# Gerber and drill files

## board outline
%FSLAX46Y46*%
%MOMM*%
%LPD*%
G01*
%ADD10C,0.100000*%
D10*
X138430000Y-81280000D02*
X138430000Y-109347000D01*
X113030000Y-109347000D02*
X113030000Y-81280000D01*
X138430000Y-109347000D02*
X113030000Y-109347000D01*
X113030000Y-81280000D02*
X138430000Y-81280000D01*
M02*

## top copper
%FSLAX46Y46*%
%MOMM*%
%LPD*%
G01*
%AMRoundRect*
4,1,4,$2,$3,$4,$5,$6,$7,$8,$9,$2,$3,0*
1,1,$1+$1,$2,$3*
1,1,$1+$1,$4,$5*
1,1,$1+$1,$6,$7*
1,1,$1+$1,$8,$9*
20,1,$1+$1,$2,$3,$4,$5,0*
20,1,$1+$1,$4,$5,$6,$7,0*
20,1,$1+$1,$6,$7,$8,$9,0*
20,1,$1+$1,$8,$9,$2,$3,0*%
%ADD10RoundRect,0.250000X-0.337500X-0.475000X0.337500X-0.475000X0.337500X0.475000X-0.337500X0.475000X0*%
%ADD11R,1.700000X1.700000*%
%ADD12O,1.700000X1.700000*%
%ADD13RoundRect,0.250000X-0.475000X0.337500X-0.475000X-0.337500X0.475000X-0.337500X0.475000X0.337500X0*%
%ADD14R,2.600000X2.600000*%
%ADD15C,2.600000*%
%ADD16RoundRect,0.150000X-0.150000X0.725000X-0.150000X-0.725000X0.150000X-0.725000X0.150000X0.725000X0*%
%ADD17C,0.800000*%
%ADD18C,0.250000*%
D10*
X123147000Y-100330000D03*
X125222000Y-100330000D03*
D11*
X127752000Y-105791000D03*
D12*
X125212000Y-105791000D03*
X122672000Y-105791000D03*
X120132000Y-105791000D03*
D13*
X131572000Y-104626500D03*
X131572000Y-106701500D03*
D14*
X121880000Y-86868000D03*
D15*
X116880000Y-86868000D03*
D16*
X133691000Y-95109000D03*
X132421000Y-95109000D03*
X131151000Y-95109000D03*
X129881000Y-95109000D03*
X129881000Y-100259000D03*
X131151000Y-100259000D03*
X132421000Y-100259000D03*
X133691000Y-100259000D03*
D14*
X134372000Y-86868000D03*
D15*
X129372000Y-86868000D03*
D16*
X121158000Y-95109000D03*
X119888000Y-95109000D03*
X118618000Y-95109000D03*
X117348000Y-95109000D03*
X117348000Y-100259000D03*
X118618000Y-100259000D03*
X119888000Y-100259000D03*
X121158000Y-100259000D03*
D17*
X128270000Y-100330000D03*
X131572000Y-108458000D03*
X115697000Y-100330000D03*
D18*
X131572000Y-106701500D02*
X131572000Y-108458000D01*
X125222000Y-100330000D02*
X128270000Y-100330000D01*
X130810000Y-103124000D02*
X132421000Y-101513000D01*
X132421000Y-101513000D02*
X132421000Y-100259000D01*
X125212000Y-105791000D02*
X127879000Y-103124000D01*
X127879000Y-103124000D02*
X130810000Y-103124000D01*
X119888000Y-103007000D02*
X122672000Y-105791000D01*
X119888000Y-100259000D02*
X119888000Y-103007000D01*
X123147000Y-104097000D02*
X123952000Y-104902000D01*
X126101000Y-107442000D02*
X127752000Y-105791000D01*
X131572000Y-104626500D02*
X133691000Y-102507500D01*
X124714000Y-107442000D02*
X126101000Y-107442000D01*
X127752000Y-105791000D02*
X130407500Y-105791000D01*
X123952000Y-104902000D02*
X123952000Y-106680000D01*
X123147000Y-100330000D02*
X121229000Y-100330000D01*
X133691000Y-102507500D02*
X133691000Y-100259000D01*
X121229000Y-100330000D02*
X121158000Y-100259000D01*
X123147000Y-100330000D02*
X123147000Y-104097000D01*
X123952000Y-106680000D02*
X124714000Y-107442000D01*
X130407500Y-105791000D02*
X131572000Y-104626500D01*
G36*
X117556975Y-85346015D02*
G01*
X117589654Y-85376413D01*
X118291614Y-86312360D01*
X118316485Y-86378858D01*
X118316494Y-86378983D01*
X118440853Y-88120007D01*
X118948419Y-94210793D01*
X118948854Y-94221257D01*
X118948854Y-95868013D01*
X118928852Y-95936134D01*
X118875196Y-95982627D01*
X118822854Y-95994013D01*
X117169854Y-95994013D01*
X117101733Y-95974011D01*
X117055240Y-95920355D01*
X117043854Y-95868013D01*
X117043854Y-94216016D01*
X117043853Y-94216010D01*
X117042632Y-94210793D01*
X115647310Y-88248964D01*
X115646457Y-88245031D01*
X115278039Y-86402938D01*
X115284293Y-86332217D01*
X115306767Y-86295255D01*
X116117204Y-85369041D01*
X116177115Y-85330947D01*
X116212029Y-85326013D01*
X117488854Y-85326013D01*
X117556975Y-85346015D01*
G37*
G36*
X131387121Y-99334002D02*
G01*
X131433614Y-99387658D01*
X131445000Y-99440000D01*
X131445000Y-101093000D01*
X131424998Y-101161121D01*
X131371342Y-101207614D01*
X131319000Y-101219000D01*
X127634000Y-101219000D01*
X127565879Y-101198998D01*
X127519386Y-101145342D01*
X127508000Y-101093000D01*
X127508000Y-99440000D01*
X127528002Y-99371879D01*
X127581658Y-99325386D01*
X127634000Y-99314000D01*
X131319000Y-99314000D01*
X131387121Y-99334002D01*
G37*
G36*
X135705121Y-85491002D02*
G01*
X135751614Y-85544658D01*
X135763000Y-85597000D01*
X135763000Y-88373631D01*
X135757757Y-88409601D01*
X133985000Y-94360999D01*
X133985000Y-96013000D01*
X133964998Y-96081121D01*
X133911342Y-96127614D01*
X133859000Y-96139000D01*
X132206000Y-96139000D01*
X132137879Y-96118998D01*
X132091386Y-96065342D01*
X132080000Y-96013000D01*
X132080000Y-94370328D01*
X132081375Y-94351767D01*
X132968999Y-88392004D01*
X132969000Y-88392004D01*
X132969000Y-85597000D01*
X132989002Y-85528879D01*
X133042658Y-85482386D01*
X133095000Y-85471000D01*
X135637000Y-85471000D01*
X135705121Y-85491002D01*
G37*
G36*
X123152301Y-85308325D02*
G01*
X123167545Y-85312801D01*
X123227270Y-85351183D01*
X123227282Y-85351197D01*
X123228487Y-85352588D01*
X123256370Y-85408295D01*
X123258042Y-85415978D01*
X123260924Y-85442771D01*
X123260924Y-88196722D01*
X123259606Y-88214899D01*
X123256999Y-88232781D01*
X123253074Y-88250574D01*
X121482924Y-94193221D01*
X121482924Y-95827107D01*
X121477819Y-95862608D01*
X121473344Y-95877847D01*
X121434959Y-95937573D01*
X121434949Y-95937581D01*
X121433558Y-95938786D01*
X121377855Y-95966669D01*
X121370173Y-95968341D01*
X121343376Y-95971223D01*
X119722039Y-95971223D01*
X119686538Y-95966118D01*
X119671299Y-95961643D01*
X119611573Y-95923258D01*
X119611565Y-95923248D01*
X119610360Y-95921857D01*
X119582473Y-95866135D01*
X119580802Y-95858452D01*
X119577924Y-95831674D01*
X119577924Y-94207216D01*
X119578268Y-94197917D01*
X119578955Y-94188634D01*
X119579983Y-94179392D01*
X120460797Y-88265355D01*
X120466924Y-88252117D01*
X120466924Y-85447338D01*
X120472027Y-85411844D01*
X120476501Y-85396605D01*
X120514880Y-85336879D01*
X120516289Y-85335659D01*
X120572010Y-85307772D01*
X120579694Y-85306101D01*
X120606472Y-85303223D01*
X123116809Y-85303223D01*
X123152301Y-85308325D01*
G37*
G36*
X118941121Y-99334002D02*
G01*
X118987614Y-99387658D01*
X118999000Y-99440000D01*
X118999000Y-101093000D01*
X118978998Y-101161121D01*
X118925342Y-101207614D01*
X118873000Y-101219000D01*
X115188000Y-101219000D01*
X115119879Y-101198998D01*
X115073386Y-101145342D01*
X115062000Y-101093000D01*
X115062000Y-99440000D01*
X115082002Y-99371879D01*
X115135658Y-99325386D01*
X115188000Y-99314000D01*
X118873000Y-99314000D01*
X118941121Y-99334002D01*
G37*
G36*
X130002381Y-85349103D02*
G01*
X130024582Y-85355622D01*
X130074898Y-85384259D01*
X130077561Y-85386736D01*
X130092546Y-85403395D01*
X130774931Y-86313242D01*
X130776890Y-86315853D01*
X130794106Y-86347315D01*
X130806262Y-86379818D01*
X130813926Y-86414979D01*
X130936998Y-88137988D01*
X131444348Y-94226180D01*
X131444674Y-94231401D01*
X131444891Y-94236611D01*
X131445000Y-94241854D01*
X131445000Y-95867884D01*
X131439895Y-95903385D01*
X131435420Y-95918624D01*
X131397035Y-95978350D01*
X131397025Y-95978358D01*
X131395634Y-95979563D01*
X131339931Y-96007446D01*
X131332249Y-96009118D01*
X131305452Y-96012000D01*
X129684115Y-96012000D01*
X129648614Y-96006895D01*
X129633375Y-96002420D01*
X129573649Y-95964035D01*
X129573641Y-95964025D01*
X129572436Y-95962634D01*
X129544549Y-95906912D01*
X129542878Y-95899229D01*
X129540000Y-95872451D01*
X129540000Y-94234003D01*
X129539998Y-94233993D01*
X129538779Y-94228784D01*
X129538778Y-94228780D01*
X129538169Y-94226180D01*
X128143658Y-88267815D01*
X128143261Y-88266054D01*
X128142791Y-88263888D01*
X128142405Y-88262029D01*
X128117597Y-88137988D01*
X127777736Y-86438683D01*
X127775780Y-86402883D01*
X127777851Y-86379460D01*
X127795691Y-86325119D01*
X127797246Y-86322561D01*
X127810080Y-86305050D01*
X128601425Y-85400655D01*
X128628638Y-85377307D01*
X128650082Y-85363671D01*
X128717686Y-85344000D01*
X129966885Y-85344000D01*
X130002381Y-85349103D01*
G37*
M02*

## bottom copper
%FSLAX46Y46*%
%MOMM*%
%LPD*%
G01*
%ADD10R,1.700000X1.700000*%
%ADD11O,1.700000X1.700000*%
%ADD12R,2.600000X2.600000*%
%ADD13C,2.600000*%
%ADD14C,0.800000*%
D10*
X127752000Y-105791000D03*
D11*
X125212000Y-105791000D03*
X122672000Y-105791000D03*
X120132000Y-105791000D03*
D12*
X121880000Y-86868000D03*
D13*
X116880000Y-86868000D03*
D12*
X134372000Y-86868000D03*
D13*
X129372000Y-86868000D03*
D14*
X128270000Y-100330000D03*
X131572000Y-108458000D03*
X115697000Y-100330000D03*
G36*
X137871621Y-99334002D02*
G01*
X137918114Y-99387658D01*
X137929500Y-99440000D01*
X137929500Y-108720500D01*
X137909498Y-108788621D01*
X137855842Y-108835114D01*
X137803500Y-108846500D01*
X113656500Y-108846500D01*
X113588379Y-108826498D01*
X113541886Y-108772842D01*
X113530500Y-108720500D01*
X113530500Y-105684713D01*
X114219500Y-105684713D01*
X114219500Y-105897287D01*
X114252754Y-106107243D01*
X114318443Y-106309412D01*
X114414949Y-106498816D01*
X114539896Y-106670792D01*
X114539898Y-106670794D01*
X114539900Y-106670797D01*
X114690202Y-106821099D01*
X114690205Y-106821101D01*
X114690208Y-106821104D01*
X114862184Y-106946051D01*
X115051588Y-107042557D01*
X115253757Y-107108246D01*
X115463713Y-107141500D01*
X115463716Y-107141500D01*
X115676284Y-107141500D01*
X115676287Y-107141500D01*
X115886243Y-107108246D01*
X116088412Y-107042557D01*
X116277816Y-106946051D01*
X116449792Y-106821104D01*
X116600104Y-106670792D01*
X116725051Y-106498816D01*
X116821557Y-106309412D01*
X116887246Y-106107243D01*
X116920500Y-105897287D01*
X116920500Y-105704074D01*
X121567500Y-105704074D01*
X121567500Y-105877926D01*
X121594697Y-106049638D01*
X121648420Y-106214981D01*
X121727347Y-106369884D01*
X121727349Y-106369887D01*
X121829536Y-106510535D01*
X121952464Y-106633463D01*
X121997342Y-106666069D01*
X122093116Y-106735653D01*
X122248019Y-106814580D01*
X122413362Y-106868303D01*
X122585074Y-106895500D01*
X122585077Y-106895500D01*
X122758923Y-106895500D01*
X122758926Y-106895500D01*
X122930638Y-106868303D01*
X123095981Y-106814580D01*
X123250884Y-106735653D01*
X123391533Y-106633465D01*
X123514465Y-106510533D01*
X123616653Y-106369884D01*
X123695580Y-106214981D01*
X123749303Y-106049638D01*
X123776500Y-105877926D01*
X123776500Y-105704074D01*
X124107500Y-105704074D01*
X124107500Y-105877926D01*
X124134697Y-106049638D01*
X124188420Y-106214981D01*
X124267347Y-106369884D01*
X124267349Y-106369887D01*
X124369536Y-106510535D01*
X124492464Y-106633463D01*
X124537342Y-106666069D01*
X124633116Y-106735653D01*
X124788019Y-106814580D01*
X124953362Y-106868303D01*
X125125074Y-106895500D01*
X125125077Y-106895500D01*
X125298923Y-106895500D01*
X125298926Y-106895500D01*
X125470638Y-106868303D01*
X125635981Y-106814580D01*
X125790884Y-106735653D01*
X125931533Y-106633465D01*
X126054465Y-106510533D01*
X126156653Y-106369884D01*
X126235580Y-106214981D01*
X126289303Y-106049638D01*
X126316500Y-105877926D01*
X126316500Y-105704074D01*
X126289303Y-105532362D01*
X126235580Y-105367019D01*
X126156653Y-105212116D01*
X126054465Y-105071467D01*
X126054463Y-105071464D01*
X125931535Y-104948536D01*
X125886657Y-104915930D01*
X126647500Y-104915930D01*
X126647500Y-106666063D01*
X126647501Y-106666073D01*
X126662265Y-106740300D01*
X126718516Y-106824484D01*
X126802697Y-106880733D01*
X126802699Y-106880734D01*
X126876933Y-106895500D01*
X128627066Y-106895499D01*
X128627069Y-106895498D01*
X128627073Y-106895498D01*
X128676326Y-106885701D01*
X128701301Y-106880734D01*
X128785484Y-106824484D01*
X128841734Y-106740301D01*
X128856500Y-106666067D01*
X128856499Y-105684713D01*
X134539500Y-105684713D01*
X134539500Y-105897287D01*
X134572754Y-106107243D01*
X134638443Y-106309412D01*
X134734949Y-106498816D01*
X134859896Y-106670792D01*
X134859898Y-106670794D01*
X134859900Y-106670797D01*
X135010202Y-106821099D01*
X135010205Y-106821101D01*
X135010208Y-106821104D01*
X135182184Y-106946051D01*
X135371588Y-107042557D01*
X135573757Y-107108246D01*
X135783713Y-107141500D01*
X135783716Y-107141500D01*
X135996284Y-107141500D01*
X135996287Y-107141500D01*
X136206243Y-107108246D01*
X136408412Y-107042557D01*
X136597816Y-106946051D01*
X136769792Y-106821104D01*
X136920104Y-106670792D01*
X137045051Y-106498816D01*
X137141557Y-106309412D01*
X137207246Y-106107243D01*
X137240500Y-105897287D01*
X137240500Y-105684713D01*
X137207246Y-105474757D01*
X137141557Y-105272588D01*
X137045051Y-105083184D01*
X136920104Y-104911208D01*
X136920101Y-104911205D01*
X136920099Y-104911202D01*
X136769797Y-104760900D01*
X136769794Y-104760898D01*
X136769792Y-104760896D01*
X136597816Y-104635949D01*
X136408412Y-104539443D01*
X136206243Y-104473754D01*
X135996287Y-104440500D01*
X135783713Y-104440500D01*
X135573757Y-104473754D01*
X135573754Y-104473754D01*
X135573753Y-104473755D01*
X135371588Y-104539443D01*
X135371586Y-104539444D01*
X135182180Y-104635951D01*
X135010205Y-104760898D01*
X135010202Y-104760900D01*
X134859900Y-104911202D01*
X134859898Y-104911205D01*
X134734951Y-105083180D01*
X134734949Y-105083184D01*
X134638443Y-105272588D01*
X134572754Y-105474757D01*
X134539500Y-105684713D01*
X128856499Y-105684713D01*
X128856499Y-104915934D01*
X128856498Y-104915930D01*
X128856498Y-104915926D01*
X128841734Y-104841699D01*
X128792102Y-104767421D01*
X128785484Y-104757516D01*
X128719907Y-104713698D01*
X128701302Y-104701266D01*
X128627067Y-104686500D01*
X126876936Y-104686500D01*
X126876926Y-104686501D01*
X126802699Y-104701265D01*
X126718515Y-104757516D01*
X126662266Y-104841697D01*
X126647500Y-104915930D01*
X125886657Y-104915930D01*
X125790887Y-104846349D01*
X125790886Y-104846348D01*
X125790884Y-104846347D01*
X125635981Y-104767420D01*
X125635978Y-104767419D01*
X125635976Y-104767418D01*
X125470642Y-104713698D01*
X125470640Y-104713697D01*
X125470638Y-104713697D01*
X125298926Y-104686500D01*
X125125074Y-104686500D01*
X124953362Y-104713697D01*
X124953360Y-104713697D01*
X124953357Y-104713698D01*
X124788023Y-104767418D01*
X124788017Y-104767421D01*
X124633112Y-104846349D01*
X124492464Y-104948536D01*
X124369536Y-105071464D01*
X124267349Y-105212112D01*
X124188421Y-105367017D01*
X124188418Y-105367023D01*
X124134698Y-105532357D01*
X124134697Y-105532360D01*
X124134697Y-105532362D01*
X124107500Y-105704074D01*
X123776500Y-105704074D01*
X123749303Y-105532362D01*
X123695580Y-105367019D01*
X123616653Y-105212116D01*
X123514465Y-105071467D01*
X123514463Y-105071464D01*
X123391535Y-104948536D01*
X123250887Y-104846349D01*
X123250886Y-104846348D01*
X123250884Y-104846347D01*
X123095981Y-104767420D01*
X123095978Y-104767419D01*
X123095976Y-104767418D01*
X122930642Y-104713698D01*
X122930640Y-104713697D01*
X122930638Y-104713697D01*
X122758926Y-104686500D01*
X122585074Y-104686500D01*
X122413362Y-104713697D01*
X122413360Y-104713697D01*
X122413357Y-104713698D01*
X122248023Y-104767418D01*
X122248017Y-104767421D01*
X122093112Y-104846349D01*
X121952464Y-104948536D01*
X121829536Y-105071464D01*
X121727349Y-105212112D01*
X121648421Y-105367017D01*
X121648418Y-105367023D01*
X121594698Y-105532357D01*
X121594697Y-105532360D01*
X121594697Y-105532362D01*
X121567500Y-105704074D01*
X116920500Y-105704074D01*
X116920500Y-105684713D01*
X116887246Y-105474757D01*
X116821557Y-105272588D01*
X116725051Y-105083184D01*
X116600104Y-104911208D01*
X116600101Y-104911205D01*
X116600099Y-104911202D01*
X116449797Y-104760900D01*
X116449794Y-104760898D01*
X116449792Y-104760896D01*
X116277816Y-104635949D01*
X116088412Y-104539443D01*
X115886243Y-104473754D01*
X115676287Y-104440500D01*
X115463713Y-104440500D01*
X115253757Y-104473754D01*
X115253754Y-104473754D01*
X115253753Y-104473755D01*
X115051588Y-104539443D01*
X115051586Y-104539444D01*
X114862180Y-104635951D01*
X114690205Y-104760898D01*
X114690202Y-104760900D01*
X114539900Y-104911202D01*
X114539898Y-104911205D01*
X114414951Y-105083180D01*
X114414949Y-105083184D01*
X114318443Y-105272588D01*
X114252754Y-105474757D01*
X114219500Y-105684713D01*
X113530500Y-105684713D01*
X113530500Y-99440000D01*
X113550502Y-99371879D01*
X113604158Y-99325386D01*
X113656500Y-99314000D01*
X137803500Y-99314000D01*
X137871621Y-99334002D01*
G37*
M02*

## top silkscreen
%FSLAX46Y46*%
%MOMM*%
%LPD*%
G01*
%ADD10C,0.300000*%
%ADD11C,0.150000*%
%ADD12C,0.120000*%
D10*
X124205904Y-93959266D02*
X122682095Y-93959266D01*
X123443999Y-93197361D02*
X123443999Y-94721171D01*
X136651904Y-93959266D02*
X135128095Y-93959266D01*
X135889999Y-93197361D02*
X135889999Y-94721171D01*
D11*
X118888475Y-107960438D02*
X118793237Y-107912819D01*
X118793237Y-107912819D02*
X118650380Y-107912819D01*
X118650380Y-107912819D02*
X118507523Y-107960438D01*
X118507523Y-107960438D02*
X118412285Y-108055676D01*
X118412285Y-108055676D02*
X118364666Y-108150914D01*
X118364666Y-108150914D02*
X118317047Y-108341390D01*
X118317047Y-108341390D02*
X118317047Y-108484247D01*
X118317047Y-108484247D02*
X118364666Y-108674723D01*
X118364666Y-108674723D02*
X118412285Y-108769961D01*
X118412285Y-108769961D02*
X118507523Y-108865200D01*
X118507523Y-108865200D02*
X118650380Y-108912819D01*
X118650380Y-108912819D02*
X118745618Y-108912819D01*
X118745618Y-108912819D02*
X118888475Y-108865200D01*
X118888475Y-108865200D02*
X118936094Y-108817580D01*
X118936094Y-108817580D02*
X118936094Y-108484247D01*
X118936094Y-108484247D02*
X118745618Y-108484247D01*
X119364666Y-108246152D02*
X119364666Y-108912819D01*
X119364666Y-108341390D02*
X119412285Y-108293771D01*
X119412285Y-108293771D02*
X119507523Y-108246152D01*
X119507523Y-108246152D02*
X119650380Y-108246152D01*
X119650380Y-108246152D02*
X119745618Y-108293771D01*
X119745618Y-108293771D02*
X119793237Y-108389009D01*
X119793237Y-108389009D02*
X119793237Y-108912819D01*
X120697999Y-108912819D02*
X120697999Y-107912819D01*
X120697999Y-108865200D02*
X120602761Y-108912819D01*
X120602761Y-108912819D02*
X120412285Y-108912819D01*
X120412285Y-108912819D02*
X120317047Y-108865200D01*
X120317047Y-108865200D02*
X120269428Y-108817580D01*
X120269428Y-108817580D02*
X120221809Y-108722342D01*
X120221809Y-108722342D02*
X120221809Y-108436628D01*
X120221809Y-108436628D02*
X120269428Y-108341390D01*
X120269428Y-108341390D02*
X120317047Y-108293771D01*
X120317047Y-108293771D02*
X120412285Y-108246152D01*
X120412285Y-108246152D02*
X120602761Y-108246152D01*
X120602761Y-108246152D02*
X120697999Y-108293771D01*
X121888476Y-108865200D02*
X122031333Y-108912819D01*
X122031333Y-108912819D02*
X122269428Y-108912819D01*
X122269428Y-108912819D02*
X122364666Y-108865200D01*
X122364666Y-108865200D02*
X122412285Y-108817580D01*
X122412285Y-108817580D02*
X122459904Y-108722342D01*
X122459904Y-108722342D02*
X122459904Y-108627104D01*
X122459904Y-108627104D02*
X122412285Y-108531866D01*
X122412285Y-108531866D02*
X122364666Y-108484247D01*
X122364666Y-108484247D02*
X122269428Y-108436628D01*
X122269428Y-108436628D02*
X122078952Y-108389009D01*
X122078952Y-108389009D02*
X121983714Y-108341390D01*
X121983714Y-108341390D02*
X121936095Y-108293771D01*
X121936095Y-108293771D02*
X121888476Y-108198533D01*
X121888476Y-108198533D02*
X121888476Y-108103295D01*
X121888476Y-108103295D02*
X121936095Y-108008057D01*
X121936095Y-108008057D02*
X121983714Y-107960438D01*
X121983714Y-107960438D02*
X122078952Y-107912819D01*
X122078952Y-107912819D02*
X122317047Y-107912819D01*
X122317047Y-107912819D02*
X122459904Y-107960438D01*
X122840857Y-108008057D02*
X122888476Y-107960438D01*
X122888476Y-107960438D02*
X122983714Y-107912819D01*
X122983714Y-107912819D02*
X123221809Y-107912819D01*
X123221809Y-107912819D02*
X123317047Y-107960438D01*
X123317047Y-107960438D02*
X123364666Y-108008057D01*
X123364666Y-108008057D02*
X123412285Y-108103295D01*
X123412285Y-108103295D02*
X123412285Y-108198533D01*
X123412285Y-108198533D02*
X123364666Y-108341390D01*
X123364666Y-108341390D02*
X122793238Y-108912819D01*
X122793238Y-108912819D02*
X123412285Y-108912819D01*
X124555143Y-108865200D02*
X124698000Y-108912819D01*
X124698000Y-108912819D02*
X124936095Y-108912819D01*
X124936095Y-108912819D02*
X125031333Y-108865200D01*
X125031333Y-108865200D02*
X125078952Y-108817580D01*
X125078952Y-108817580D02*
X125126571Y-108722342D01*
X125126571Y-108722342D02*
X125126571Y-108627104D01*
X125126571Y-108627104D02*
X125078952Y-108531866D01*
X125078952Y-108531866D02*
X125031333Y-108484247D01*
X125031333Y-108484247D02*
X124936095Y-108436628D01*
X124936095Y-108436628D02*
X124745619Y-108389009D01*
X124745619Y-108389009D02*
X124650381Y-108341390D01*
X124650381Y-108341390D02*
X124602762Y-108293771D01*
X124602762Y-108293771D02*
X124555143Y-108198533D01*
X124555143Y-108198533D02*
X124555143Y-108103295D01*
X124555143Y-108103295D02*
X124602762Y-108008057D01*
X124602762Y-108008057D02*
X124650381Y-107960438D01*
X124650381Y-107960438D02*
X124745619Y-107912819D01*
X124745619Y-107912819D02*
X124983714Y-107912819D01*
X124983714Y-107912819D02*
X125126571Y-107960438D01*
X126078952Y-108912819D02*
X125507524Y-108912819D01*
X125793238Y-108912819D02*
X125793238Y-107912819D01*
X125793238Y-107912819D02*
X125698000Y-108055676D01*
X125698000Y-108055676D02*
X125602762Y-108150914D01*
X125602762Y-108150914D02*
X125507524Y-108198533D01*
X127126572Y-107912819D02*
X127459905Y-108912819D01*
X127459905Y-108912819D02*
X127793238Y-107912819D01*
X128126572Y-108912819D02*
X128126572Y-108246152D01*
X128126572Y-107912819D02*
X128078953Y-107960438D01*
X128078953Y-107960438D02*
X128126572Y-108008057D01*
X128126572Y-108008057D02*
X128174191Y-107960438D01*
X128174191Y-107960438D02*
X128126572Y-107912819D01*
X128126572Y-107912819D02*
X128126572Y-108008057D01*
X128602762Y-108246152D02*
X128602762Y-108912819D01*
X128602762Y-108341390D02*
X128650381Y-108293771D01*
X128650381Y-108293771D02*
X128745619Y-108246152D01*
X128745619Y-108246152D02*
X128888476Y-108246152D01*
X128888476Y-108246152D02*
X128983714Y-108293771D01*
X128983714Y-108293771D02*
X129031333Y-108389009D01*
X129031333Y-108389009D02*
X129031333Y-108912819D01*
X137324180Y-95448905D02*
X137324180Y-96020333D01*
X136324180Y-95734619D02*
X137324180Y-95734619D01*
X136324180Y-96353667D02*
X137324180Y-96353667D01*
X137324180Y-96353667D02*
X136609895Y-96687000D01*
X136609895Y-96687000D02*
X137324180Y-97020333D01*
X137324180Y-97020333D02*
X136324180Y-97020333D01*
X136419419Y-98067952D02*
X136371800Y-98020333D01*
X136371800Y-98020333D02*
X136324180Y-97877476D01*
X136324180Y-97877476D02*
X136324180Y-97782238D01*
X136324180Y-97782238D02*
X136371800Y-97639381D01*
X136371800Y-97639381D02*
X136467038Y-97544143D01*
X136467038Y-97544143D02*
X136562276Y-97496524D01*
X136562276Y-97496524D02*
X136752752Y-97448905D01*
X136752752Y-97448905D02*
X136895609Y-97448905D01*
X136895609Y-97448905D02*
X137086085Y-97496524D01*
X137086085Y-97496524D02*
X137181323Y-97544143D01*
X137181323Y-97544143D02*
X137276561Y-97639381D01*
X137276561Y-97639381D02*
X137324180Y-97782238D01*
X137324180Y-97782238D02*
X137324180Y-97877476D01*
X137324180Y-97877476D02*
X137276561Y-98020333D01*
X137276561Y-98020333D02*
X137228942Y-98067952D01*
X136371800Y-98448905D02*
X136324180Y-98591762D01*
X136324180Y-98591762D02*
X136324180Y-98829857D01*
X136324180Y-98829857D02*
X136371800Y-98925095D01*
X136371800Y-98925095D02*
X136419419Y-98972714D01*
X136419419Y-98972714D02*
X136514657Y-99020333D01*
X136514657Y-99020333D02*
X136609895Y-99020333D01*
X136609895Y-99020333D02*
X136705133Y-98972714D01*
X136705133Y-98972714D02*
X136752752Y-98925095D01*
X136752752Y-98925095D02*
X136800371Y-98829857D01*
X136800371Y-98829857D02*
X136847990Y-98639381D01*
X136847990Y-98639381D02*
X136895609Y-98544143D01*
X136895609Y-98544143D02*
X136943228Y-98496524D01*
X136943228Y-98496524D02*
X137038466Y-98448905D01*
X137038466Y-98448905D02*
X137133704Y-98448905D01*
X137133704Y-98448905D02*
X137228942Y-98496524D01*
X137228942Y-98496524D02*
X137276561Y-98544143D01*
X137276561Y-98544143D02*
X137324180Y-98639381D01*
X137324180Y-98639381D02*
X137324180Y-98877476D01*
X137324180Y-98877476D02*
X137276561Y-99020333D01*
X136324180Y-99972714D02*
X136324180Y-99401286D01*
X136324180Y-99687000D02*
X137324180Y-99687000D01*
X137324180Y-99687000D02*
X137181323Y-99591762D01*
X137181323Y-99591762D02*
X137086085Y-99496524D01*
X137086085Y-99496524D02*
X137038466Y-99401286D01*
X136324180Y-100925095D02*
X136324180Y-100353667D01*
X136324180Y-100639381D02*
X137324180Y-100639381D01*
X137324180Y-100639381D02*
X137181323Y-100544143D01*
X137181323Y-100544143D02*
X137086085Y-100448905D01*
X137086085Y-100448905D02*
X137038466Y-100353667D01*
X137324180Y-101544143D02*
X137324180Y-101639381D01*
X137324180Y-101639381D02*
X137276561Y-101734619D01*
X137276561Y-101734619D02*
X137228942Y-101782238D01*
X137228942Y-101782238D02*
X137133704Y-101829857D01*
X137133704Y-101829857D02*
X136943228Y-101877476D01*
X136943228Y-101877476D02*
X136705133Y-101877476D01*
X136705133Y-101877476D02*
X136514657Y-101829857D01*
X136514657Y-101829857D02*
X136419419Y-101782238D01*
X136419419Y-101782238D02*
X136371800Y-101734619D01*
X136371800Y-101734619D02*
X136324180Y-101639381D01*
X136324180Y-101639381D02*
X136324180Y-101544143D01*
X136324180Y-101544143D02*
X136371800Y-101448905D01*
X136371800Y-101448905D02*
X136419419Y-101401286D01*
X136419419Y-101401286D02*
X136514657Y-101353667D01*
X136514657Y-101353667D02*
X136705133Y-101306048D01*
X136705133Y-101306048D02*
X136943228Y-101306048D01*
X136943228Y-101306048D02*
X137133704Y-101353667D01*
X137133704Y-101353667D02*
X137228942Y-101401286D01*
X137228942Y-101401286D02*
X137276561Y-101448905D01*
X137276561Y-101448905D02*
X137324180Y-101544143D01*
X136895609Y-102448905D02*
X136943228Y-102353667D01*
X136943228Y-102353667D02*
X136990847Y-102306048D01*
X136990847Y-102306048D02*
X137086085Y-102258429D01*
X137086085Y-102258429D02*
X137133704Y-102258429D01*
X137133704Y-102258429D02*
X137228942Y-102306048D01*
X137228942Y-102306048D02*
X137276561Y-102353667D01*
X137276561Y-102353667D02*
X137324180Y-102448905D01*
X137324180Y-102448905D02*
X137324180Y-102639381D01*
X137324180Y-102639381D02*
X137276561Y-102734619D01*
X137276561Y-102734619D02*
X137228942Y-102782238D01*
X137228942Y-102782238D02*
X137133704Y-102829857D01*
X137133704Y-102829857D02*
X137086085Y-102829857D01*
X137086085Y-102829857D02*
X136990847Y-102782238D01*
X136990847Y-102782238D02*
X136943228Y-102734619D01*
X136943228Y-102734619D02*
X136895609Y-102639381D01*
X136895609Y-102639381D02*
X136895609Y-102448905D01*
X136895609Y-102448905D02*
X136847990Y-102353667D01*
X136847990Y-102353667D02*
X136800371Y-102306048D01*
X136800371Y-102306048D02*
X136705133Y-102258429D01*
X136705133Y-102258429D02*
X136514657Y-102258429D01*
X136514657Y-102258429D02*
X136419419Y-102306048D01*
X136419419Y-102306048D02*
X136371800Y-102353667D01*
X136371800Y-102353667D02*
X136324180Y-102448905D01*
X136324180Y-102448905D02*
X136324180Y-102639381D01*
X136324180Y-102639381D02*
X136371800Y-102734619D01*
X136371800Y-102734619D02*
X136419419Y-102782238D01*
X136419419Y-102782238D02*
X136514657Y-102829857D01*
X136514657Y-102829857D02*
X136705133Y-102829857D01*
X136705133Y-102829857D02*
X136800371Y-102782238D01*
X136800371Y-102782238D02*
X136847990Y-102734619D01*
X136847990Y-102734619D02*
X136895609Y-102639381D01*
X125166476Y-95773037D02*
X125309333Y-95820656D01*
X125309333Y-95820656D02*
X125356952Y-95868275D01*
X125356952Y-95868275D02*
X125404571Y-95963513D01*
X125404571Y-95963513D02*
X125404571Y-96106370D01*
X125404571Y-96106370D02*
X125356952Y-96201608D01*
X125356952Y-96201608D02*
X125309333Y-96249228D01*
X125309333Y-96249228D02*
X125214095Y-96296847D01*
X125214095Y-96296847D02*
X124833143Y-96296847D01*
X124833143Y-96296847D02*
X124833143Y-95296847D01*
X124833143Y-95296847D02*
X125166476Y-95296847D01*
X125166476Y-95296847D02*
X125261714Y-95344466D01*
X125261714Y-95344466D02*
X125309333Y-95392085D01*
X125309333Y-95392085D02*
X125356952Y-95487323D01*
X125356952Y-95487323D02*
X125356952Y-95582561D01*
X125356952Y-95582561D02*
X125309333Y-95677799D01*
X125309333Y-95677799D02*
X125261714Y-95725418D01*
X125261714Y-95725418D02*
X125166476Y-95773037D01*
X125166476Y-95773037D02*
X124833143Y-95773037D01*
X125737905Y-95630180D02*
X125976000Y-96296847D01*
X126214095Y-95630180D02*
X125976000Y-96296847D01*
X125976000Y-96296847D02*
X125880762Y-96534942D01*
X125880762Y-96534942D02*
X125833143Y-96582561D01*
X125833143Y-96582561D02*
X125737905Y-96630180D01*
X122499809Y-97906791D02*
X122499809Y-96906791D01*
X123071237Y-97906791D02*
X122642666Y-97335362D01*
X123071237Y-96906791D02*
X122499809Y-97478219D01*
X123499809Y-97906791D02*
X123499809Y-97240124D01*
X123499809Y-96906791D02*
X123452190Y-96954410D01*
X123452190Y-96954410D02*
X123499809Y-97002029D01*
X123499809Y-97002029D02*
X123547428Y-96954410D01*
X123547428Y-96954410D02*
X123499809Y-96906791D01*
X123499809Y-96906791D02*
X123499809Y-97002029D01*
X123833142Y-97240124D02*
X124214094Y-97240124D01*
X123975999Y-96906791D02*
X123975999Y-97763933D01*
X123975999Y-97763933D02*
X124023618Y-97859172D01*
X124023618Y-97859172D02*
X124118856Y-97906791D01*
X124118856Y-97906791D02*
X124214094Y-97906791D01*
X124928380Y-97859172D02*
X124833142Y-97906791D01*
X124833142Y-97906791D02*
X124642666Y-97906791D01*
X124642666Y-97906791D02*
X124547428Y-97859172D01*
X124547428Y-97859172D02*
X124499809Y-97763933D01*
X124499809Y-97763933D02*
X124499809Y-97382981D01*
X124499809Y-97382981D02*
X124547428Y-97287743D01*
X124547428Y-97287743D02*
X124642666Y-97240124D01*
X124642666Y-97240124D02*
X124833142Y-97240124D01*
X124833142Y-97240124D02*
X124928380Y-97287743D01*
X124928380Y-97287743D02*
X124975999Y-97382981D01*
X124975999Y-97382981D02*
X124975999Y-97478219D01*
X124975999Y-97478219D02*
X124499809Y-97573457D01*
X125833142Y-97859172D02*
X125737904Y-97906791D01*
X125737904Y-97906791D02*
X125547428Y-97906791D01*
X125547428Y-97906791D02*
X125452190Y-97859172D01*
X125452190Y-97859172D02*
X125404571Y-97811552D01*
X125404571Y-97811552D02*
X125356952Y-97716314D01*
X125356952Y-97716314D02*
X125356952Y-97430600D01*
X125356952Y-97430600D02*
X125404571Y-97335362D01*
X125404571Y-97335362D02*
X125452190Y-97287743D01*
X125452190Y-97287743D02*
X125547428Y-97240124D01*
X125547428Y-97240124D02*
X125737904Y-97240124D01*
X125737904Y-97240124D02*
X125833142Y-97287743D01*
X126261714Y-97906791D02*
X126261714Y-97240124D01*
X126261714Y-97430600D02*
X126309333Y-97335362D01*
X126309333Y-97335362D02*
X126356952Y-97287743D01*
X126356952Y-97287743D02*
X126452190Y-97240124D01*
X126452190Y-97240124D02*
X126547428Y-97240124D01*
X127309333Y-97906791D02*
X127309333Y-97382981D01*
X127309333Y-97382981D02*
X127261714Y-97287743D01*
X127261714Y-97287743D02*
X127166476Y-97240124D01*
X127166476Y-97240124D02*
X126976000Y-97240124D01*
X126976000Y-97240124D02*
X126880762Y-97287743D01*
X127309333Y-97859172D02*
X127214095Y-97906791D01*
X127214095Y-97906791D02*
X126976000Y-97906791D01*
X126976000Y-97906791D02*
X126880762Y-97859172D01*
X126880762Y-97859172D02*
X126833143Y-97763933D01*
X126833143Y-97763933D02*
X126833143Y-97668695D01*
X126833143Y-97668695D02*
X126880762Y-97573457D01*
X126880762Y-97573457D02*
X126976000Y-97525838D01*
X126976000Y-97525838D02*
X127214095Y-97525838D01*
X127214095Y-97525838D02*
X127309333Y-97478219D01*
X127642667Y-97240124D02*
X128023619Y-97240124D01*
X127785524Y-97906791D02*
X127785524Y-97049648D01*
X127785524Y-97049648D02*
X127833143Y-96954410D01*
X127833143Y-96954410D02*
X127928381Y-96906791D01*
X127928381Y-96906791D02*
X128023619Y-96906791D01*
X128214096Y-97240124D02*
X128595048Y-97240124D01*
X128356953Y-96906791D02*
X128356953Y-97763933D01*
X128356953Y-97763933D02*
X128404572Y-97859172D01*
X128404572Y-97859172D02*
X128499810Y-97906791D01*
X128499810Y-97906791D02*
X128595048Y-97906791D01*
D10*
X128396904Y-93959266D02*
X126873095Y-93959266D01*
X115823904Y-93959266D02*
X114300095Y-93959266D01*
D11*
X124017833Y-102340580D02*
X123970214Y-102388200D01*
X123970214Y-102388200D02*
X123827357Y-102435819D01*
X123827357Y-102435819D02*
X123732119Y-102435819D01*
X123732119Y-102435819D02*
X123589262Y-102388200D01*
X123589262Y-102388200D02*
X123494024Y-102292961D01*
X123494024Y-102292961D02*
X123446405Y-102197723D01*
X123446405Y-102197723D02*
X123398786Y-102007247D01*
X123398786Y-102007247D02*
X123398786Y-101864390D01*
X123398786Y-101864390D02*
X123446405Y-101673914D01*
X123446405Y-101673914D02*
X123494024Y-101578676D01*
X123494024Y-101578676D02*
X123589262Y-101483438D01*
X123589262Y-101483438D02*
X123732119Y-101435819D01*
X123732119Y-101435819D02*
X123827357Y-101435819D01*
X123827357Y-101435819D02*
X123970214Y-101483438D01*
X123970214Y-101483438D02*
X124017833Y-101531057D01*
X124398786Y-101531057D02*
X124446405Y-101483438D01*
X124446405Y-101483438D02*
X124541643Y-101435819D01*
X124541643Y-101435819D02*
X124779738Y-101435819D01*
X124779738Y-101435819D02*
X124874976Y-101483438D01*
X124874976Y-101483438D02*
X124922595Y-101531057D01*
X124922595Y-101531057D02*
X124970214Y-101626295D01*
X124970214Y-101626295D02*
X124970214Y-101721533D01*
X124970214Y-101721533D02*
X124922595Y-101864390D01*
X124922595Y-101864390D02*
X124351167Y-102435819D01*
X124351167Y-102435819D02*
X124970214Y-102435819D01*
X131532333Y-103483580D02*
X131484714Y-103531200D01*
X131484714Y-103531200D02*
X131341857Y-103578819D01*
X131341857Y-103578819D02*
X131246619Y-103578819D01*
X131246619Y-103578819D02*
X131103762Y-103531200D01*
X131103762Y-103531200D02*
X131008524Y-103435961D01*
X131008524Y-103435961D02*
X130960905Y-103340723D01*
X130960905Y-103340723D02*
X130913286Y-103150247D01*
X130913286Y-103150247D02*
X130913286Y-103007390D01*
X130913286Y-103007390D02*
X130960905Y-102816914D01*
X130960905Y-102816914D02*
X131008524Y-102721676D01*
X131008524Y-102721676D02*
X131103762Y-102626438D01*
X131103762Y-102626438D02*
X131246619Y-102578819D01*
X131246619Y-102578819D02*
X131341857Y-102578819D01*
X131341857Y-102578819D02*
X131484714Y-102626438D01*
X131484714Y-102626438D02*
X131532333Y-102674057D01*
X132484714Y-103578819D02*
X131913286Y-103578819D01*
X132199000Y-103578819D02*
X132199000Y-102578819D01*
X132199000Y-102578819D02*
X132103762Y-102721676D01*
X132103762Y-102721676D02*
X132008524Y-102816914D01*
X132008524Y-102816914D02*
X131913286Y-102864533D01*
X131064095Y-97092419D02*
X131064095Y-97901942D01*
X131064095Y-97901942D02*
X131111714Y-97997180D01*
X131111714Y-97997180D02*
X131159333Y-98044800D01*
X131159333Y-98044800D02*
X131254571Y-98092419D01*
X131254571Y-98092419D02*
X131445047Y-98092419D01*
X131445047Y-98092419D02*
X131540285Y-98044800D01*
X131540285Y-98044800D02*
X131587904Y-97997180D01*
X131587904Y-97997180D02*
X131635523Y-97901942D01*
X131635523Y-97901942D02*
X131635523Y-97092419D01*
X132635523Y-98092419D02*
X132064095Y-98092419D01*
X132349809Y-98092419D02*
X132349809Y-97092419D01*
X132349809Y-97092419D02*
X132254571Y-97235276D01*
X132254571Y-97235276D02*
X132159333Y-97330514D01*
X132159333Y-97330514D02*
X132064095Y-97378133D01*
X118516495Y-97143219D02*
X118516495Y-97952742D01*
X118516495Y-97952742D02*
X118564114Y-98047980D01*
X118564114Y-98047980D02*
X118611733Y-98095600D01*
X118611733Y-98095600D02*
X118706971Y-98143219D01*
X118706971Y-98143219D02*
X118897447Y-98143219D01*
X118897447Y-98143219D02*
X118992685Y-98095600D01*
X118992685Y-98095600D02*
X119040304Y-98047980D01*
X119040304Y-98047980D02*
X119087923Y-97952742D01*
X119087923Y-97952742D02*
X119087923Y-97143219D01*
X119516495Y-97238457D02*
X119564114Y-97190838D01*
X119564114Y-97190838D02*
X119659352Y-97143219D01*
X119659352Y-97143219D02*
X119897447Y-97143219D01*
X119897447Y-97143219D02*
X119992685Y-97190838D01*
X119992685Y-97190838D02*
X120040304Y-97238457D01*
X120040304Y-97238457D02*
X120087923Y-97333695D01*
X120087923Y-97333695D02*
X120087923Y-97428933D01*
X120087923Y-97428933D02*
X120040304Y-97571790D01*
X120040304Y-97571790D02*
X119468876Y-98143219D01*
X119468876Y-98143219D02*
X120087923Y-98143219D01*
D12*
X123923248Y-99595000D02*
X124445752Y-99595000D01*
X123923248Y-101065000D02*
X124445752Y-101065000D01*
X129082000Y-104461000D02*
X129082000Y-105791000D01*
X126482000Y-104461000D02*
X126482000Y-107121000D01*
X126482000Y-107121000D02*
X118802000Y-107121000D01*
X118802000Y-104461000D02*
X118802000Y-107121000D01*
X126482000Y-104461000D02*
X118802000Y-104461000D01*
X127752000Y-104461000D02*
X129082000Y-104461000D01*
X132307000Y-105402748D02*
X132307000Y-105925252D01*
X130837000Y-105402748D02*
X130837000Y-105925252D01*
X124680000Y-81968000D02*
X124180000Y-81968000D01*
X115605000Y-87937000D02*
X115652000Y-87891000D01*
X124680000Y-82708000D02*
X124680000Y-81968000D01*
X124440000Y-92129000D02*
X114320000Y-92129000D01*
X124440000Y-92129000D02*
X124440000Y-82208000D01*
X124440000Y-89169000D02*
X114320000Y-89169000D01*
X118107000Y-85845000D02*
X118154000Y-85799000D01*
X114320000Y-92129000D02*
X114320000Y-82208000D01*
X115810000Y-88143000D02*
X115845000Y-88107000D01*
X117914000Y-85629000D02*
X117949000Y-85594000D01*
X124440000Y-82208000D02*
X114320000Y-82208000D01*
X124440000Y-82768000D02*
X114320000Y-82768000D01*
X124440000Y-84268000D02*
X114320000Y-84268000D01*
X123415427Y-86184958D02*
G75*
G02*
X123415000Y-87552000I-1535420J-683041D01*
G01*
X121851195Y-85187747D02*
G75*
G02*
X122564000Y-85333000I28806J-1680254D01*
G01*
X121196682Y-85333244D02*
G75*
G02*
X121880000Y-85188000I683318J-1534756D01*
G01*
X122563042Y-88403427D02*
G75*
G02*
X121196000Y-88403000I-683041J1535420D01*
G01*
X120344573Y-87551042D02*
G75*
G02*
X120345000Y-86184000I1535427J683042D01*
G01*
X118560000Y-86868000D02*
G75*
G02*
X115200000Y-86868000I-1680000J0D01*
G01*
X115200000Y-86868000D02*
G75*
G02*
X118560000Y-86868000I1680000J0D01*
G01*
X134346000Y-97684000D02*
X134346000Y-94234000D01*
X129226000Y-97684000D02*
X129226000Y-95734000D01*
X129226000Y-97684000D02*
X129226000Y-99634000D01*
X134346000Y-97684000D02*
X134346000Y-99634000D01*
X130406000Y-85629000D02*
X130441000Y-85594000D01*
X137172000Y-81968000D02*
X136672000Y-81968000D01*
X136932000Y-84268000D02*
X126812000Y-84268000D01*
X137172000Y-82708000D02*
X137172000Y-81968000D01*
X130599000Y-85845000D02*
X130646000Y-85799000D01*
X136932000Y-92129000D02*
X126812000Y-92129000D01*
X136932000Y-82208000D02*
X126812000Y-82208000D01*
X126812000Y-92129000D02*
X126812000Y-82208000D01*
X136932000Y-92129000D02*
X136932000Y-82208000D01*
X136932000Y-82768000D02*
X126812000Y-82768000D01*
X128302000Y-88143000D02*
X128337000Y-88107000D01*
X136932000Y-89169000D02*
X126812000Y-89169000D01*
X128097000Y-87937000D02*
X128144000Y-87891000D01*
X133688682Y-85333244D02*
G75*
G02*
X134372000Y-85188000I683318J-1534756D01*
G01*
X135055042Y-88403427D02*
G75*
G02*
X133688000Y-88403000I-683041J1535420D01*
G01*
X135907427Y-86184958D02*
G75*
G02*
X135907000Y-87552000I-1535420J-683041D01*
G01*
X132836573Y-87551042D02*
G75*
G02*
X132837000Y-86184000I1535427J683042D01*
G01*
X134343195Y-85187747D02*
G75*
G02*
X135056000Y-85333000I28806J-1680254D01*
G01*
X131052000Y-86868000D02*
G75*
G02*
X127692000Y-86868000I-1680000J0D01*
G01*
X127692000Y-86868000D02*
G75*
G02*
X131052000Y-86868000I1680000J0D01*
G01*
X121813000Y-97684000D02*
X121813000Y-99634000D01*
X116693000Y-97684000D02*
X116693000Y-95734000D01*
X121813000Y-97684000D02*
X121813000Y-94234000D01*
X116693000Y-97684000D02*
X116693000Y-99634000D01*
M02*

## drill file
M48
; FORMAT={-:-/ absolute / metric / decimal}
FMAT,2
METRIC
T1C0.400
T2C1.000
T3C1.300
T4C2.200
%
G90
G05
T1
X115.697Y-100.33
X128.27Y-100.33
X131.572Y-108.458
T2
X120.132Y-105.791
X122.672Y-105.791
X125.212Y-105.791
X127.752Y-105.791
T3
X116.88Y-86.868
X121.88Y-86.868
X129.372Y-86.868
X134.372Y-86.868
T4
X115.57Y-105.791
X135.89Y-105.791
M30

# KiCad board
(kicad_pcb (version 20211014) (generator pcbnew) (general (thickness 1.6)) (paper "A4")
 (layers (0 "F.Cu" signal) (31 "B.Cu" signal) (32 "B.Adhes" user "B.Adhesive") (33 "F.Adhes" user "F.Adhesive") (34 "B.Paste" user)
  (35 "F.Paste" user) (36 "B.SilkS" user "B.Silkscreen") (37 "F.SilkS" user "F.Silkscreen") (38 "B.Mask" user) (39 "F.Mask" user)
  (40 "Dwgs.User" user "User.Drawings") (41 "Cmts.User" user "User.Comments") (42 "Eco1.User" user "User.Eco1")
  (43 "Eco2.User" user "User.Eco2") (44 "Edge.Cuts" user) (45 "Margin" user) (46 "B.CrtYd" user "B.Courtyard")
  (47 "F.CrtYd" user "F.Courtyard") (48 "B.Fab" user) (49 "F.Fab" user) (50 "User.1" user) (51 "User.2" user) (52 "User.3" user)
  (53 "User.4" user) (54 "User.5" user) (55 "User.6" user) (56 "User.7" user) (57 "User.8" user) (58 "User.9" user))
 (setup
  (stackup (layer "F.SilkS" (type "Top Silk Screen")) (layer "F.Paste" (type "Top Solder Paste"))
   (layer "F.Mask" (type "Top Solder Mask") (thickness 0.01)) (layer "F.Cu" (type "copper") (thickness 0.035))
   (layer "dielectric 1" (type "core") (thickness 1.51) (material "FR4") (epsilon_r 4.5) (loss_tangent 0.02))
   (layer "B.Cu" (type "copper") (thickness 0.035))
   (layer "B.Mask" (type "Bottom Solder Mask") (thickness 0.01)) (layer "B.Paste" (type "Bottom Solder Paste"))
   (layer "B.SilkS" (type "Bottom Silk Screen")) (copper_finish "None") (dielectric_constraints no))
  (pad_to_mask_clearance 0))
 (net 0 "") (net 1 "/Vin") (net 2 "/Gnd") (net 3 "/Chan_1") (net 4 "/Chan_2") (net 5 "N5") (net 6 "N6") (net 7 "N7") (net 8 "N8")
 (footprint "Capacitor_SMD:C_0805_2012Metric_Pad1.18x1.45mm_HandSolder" (layer "F.Cu") (at 124.1845 100.33)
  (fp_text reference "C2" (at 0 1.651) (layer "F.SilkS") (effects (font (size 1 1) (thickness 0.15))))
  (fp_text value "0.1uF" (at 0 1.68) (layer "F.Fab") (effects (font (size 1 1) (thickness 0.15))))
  (fp_line (start -0.261252 -0.735) (end 0.261252 -0.735) (layer "F.SilkS") (width 0.12))
  (fp_line (start -0.261252 0.735) (end 0.261252 0.735) (layer "F.SilkS") (width 0.12))
  (pad "1" smd roundrect (at -1.0375 0) (size 1.175 1.45) (layers "F.Cu" "F.Paste" "F.Mask") (roundrect_rratio 0.212766) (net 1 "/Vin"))
  (pad "2" smd roundrect (at 1.0375 0) (size 1.175 1.45) (layers "F.Cu" "F.Paste" "F.Mask") (roundrect_rratio 0.212766) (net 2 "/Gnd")))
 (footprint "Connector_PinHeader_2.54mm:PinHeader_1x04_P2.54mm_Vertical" (layer "F.Cu") (at 127.752 105.791 -90)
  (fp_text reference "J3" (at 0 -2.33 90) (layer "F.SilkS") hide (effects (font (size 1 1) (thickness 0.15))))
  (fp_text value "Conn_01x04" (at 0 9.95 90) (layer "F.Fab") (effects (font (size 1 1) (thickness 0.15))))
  (fp_line (start -1.33 -1.33) (end 0 -1.33) (layer "F.SilkS") (width 0.12))
  (fp_line (start -1.33 1.27) (end 1.33 1.27) (layer "F.SilkS") (width 0.12))
  (fp_line (start 1.33 1.27) (end 1.33 8.95) (layer "F.SilkS") (width 0.12))
  (fp_line (start -1.33 8.95) (end 1.33 8.95) (layer "F.SilkS") (width 0.12))
  (fp_line (start -1.33 1.27) (end -1.33 8.95) (layer "F.SilkS") (width 0.12))
  (fp_line (start -1.33 0) (end -1.33 -1.33) (layer "F.SilkS") (width 0.12))
  (pad "1" thru_hole rect (at 0 0 270) (size 1.7 1.7) (drill 1) (layers *.Cu *.Mask) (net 1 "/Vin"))
  (pad "2" thru_hole oval (at 0 2.54 270) (size 1.7 1.7) (drill 1) (layers *.Cu *.Mask) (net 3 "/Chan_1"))
  (pad "3" thru_hole oval (at 0 5.08 270) (size 1.7 1.7) (drill 1) (layers *.Cu *.Mask) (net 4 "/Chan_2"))
  (pad "4" thru_hole oval (at 0 7.62 270) (size 1.7 1.7) (drill 1) (layers *.Cu *.Mask) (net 2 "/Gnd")))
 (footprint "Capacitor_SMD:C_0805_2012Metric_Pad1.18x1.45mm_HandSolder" (layer "F.Cu") (at 131.572 105.664 -90)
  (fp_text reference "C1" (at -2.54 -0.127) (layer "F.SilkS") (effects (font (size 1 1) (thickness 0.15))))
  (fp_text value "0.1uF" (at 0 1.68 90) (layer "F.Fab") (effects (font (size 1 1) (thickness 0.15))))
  (fp_line (start -0.261252 -0.735) (end 0.261252 -0.735) (layer "F.SilkS") (width 0.12))
  (fp_line (start -0.261252 0.735) (end 0.261252 0.735) (layer "F.SilkS") (width 0.12))
  (pad "1" smd roundrect (at -1.0375 0 270) (size 1.175 1.45) (layers "F.Cu" "F.Paste" "F.Mask") (roundrect_rratio 0.212766) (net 1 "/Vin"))
  (pad "2" smd roundrect (at 1.0375 0 270) (size 1.175 1.45) (layers "F.Cu" "F.Paste" "F.Mask") (roundrect_rratio 0.212766) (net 2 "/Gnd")))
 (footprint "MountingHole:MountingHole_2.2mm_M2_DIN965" (layer "F.Cu") (at 135.89 105.791)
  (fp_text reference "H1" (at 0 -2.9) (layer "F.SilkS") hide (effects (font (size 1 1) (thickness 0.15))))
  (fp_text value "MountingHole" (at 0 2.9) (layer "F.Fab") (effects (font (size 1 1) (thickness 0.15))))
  (pad "" np_thru_hole circle (at 0 0) (size 2.2 2.2) (drill 2.2) (layers *.Cu *.Mask)))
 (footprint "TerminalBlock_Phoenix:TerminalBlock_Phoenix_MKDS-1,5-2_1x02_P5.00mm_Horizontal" (layer "F.Cu") (at 121.88 86.868 180)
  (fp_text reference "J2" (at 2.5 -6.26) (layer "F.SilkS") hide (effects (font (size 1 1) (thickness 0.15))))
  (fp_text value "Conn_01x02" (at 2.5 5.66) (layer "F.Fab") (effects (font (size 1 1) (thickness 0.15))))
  (fp_line (start -2.8 4.9) (end -2.3 4.9) (layer "F.SilkS") (width 0.12))
  (fp_line (start 6.275 -1.069) (end 6.228 -1.023) (layer "F.SilkS") (width 0.12))
  (fp_line (start -2.8 4.16) (end -2.8 4.9) (layer "F.SilkS") (width 0.12))
  (fp_line (start -2.56 -5.261) (end 7.56 -5.261) (layer "F.SilkS") (width 0.12))
  (fp_line (start -2.56 -5.261) (end -2.56 4.66) (layer "F.SilkS") (width 0.12))
  (fp_line (start -2.56 -2.301) (end 7.56 -2.301) (layer "F.SilkS") (width 0.12))
  (fp_line (start 3.773 1.023) (end 3.726 1.069) (layer "F.SilkS") (width 0.12))
  (fp_line (start 7.56 -5.261) (end 7.56 4.66) (layer "F.SilkS") (width 0.12))
  (fp_line (start 6.07 -1.275) (end 6.035 -1.239) (layer "F.SilkS") (width 0.12))
  (fp_line (start 3.966 1.239) (end 3.931 1.274) (layer "F.SilkS") (width 0.12))
  (fp_line (start -2.56 4.66) (end 7.56 4.66) (layer "F.SilkS") (width 0.12))
  (fp_line (start -2.56 4.1) (end 7.56 4.1) (layer "F.SilkS") (width 0.12))
  (fp_line (start -2.56 2.6) (end 7.56 2.6) (layer "F.SilkS") (width 0.12))
  (fp_arc (start -1.535427 0.683042) (mid -1.680501 -0.000524) (end -1.535 -0.684) (layer "F.SilkS") (width 0.12))
  (fp_arc (start 0.028805 1.680253) (mid -0.335551 1.646659) (end -0.684 1.535) (layer "F.SilkS") (width 0.12))
  (fp_arc (start 0.683318 1.534756) (mid 0.349292 1.643288) (end 0 1.68) (layer "F.SilkS") (width 0.12))
  (fp_arc (start -0.683042 -1.535427) (mid 0.000524 -1.680501) (end 0.684 -1.535) (layer "F.SilkS") (width 0.12))
  (fp_arc (start 1.535427 -0.683042) (mid 1.680501 0.000524) (end 1.535 0.684) (layer "F.SilkS") (width 0.12))
  (fp_circle (center 5 0) (end 6.68 0) (layer "F.SilkS") (width 0.12) (fill none))
  (pad "1" thru_hole rect (at 0 0 180) (size 2.6 2.6) (drill 1.3) (layers *.Cu *.Mask) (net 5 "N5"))
  (pad "2" thru_hole circle (at 5 0 180) (size 2.6 2.6) (drill 1.3) (layers *.Cu *.Mask) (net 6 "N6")))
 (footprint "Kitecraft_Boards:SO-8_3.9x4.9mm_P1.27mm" (layer "F.Cu") (at 131.786 97.684 -90)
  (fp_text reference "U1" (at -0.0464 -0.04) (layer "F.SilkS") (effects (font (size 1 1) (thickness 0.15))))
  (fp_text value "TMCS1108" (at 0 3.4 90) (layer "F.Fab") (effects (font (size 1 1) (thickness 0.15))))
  (fp_line (start 0 -2.56) (end -3.45 -2.56) (layer "F.SilkS") (width 0.12))
  (fp_line (start 0 2.56) (end -1.95 2.56) (layer "F.SilkS") (width 0.12))
  (fp_line (start 0 2.56) (end 1.95 2.56) (layer "F.SilkS") (width 0.12))
  (fp_line (start 0 -2.56) (end 1.95 -2.56) (layer "F.SilkS") (width 0.12))
  (pad "1" smd roundrect (at -2.575 -1.905 270) (size 1.75 0.6) (layers "F.Cu" "F.Paste" "F.Mask") (roundrect_rratio 0.25) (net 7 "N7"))
  (pad "2" smd roundrect (at -2.575 -0.635 270) (size 1.75 0.6) (layers "F.Cu" "F.Paste" "F.Mask") (roundrect_rratio 0.25) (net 7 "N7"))
  (pad "3" smd roundrect (at -2.575 0.635 270) (size 1.75 0.6) (layers "F.Cu" "F.Paste" "F.Mask") (roundrect_rratio 0.25) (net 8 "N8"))
  (pad "4" smd roundrect (at -2.575 1.905 270) (size 1.75 0.6) (layers "F.Cu" "F.Paste" "F.Mask") (roundrect_rratio 0.25) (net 8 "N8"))
  (pad "5" smd roundrect (at 2.575 1.905 270) (size 1.75 0.6) (layers "F.Cu" "F.Paste" "F.Mask") (roundrect_rratio 0.25) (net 2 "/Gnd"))
  (pad "6" smd roundrect (at 2.575 0.635 270) (size 1.75 0.6) (layers "F.Cu" "F.Paste" "F.Mask") (roundrect_rratio 0.25) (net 2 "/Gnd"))
  (pad "7" smd roundrect (at 2.575 -0.635 270) (size 1.75 0.6) (layers "F.Cu" "F.Paste" "F.Mask") (roundrect_rratio 0.25) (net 3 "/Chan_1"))
  (pad "8" smd roundrect (at 2.575 -1.905 270) (size 1.75 0.6) (layers "F.Cu" "F.Paste" "F.Mask") (roundrect_rratio 0.25) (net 1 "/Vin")))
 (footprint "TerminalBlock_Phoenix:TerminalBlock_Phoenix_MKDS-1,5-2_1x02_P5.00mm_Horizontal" (layer "F.Cu") (at 134.372 86.868 180)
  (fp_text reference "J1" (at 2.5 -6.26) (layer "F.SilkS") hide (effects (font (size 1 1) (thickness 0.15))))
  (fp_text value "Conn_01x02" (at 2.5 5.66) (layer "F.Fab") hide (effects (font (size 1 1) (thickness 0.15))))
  (fp_line (start 3.966 1.239) (end 3.931 1.274) (layer "F.SilkS") (width 0.12))
  (fp_line (start -2.8 4.9) (end -2.3 4.9) (layer "F.SilkS") (width 0.12))
  (fp_line (start -2.56 2.6) (end 7.56 2.6) (layer "F.SilkS") (width 0.12))
  (fp_line (start -2.8 4.16) (end -2.8 4.9) (layer "F.SilkS") (width 0.12))
  (fp_line (start 3.773 1.023) (end 3.726 1.069) (layer "F.SilkS") (width 0.12))
  (fp_line (start -2.56 -5.261) (end 7.56 -5.261) (layer "F.SilkS") (width 0.12))
  (fp_line (start -2.56 4.66) (end 7.56 4.66) (layer "F.SilkS") (width 0.12))
  (fp_line (start 7.56 -5.261) (end 7.56 4.66) (layer "F.SilkS") (width 0.12))
  (fp_line (start -2.56 -5.261) (end -2.56 4.66) (layer "F.SilkS") (width 0.12))
  (fp_line (start -2.56 4.1) (end 7.56 4.1) (layer "F.SilkS") (width 0.12))
  (fp_line (start 6.07 -1.275) (end 6.035 -1.239) (layer "F.SilkS") (width 0.12))
  (fp_line (start -2.56 -2.301) (end 7.56 -2.301) (layer "F.SilkS") (width 0.12))
  (fp_line (start 6.275 -1.069) (end 6.228 -1.023) (layer "F.SilkS") (width 0.12))
  (fp_arc (start 0.683318 1.534756) (mid 0.349292 1.643288) (end 0 1.68) (layer "F.SilkS") (width 0.12))
  (fp_arc (start -0.683042 -1.535427) (mid 0.000524 -1.680501) (end 0.684 -1.535) (layer "F.SilkS") (width 0.12))
  (fp_arc (start -1.535427 0.683042) (mid -1.680501 -0.000524) (end -1.535 -0.684) (layer "F.SilkS") (width 0.12))
  (fp_arc (start 1.535427 -0.683042) (mid 1.680501 0.000524) (end 1.535 0.684) (layer "F.SilkS") (width 0.12))
  (fp_arc (start 0.028805 1.680253) (mid -0.335551 1.646659) (end -0.684 1.535) (layer "F.SilkS") (width 0.12))
  (fp_circle (center 5 0) (end 6.68 0) (layer "F.SilkS") (width 0.12) (fill none))
  (pad "1" thru_hole rect (at 0 0 180) (size 2.6 2.6) (drill 1.3) (layers *.Cu *.Mask) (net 7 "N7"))
  (pad "2" thru_hole circle (at 5 0 180) (size 2.6 2.6) (drill 1.3) (layers *.Cu *.Mask) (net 8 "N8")))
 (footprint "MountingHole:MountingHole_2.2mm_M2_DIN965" (layer "F.Cu") (at 115.57 105.791)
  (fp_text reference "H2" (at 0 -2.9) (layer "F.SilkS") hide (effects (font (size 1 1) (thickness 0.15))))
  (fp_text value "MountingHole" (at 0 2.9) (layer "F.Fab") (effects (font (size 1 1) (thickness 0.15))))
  (pad "" np_thru_hole circle (at 0 0) (size 2.2 2.2) (drill 2.2) (layers *.Cu *.Mask)))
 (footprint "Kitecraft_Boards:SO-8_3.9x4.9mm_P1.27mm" (layer "F.Cu") (at 119.253 97.684 -90)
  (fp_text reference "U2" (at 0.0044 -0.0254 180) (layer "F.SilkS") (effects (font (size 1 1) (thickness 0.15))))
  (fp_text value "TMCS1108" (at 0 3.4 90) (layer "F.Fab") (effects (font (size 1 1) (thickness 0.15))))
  (fp_line (start 0 -2.56) (end 1.95 -2.56) (layer "F.SilkS") (width 0.12))
  (fp_line (start 0 2.56) (end -1.95 2.56) (layer "F.SilkS") (width 0.12))
  (fp_line (start 0 -2.56) (end -3.45 -2.56) (layer "F.SilkS") (width 0.12))
  (fp_line (start 0 2.56) (end 1.95 2.56) (layer "F.SilkS") (width 0.12))
  (pad "1" smd roundrect (at -2.575 -1.905 270) (size 1.75 0.6) (layers "F.Cu" "F.Paste" "F.Mask") (roundrect_rratio 0.25) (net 5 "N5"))
  (pad "2" smd roundrect (at -2.575 -0.635 270) (size 1.75 0.6) (layers "F.Cu" "F.Paste" "F.Mask") (roundrect_rratio 0.25) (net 5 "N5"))
  (pad "3" smd roundrect (at -2.575 0.635 270) (size 1.75 0.6) (layers "F.Cu" "F.Paste" "F.Mask") (roundrect_rratio 0.25) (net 6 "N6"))
  (pad "4" smd roundrect (at -2.575 1.905 270) (size 1.75 0.6) (layers "F.Cu" "F.Paste" "F.Mask") (roundrect_rratio 0.25) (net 6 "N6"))
  (pad "5" smd roundrect (at 2.575 1.905 270) (size 1.75 0.6) (layers "F.Cu" "F.Paste" "F.Mask") (roundrect_rratio 0.25) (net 2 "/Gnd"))
  (pad "6" smd roundrect (at 2.575 0.635 270) (size 1.75 0.6) (layers "F.Cu" "F.Paste" "F.Mask") (roundrect_rratio 0.25) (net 2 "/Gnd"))
  (pad "7" smd roundrect (at 2.575 -0.635 270) (size 1.75 0.6) (layers "F.Cu" "F.Paste" "F.Mask") (roundrect_rratio 0.25) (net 4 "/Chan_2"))
  (pad "8" smd roundrect (at 2.575 -1.905 270) (size 1.75 0.6) (layers "F.Cu" "F.Paste" "F.Mask") (roundrect_rratio 0.25) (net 1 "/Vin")))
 (gr_line (start 138.43 81.28) (end 138.43 109.347) (layer "Edge.Cuts") (width 0.1))
 (gr_line (start 113.03 109.347) (end 113.03 81.28) (layer "Edge.Cuts") (width 0.1))
 (gr_line (start 138.43 109.347) (end 113.03 109.347) (layer "Edge.Cuts") (width 0.1))
 (gr_line (start 113.03 81.28) (end 138.43 81.28) (layer "Edge.Cuts") (width 0.1))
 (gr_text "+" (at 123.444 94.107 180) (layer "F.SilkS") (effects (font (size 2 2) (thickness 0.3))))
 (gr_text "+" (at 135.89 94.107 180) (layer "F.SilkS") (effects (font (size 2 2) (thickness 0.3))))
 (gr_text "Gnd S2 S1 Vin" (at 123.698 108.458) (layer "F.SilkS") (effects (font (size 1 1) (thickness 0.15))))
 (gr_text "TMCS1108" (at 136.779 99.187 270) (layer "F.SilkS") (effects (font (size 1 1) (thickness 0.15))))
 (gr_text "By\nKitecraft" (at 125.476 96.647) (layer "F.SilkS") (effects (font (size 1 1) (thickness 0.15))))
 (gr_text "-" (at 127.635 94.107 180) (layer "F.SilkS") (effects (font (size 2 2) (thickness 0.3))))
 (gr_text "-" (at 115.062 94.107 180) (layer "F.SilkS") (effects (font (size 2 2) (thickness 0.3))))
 (segment (start 131.572 106.7015) (end 131.572 108.458) (width 0.25) (layer "F.Cu") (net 2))
 (segment (start 125.222 100.33) (end 128.27 100.33) (width 0.25) (layer "F.Cu") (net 2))
 (via (at 128.27 100.33) (size 0.8) (drill 0.4) (layers "F.Cu" "B.Cu") (free) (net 2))
 (via (at 131.572 108.458) (size 0.8) (drill 0.4) (layers "F.Cu" "B.Cu") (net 2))
 (via (at 115.697 100.33) (size 0.8) (drill 0.4) (layers "F.Cu" "B.Cu") (free) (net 2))
 (segment (start 130.81 103.124) (end 132.421 101.513) (width 0.25) (layer "F.Cu") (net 3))
 (segment (start 132.421 101.513) (end 132.421 100.259) (width 0.25) (layer "F.Cu") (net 3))
 (segment (start 125.212 105.791) (end 127.879 103.124) (width 0.25) (layer "F.Cu") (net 3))
 (segment (start 127.879 103.124) (end 130.81 103.124) (width 0.25) (layer "F.Cu") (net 3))
 (segment (start 119.888 103.007) (end 122.672 105.791) (width 0.25) (layer "F.Cu") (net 4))
 (segment (start 119.888 100.259) (end 119.888 103.007) (width 0.25) (layer "F.Cu") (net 4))
 (segment (start 123.147 104.097) (end 123.952 104.902) (width 0.25) (layer "F.Cu") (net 1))
 (segment (start 126.101 107.442) (end 127.752 105.791) (width 0.25) (layer "F.Cu") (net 1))
 (segment (start 131.572 104.6265) (end 133.691 102.5075) (width 0.25) (layer "F.Cu") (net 1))
 (segment (start 124.714 107.442) (end 126.101 107.442) (width 0.25) (layer "F.Cu") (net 1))
 (segment (start 127.752 105.791) (end 130.4075 105.791) (width 0.25) (layer "F.Cu") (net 1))
 (segment (start 123.952 104.902) (end 123.952 106.68) (width 0.25) (layer "F.Cu") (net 1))
 (segment (start 123.147 100.33) (end 121.229 100.33) (width 0.25) (layer "F.Cu") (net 1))
 (segment (start 133.691 102.5075) (end 133.691 100.259) (width 0.25) (layer "F.Cu") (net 1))
 (segment (start 121.229 100.33) (end 121.158 100.259) (width 0.25) (layer "F.Cu") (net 1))
 (segment (start 123.147 100.33) (end 123.147 104.097) (width 0.25) (layer "F.Cu") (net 1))
 (segment (start 123.952 106.68) (end 124.714 107.442) (width 0.25) (layer "F.Cu") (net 1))
 (segment (start 130.4075 105.791) (end 131.572 104.6265) (width 0.25) (layer "F.Cu") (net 1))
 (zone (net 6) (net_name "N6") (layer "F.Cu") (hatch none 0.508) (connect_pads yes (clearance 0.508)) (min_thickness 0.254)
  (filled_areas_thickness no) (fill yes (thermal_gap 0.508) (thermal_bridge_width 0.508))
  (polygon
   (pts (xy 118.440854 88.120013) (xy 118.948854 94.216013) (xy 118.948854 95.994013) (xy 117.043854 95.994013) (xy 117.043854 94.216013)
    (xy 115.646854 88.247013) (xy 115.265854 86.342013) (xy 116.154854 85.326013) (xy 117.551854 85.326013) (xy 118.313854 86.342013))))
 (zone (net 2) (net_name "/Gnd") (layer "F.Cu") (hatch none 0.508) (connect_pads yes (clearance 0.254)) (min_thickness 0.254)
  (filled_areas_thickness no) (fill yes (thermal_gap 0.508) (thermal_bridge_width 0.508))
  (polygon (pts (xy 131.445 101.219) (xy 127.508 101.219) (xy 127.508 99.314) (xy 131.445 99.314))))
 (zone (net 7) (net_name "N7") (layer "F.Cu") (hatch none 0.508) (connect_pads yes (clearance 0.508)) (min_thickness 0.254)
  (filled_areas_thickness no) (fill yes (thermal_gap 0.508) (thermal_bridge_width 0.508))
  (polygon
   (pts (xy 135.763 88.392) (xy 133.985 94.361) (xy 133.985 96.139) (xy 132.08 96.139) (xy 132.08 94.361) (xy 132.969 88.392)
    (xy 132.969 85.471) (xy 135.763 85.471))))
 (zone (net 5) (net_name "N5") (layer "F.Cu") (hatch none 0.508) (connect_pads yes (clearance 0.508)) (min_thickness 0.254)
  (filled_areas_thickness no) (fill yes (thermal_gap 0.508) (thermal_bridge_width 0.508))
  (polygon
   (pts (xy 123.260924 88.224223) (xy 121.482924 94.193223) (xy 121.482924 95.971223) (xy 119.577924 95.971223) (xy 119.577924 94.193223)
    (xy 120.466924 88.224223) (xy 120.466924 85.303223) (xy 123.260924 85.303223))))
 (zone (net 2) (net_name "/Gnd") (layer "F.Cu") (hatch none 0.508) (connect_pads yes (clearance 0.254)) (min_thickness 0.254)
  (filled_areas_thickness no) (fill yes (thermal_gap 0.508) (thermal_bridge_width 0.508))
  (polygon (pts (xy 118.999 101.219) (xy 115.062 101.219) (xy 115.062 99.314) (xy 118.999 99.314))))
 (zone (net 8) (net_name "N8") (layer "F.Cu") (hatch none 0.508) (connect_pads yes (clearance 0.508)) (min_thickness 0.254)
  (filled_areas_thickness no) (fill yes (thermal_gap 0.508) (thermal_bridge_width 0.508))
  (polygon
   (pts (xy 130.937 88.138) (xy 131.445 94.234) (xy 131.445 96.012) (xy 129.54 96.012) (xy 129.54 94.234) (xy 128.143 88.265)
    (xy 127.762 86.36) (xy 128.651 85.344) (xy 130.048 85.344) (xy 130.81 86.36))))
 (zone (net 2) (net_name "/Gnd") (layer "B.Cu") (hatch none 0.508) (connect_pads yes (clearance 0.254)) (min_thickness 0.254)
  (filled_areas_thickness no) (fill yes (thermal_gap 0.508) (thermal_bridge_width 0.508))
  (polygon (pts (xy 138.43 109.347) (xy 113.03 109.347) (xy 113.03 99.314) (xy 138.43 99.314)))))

